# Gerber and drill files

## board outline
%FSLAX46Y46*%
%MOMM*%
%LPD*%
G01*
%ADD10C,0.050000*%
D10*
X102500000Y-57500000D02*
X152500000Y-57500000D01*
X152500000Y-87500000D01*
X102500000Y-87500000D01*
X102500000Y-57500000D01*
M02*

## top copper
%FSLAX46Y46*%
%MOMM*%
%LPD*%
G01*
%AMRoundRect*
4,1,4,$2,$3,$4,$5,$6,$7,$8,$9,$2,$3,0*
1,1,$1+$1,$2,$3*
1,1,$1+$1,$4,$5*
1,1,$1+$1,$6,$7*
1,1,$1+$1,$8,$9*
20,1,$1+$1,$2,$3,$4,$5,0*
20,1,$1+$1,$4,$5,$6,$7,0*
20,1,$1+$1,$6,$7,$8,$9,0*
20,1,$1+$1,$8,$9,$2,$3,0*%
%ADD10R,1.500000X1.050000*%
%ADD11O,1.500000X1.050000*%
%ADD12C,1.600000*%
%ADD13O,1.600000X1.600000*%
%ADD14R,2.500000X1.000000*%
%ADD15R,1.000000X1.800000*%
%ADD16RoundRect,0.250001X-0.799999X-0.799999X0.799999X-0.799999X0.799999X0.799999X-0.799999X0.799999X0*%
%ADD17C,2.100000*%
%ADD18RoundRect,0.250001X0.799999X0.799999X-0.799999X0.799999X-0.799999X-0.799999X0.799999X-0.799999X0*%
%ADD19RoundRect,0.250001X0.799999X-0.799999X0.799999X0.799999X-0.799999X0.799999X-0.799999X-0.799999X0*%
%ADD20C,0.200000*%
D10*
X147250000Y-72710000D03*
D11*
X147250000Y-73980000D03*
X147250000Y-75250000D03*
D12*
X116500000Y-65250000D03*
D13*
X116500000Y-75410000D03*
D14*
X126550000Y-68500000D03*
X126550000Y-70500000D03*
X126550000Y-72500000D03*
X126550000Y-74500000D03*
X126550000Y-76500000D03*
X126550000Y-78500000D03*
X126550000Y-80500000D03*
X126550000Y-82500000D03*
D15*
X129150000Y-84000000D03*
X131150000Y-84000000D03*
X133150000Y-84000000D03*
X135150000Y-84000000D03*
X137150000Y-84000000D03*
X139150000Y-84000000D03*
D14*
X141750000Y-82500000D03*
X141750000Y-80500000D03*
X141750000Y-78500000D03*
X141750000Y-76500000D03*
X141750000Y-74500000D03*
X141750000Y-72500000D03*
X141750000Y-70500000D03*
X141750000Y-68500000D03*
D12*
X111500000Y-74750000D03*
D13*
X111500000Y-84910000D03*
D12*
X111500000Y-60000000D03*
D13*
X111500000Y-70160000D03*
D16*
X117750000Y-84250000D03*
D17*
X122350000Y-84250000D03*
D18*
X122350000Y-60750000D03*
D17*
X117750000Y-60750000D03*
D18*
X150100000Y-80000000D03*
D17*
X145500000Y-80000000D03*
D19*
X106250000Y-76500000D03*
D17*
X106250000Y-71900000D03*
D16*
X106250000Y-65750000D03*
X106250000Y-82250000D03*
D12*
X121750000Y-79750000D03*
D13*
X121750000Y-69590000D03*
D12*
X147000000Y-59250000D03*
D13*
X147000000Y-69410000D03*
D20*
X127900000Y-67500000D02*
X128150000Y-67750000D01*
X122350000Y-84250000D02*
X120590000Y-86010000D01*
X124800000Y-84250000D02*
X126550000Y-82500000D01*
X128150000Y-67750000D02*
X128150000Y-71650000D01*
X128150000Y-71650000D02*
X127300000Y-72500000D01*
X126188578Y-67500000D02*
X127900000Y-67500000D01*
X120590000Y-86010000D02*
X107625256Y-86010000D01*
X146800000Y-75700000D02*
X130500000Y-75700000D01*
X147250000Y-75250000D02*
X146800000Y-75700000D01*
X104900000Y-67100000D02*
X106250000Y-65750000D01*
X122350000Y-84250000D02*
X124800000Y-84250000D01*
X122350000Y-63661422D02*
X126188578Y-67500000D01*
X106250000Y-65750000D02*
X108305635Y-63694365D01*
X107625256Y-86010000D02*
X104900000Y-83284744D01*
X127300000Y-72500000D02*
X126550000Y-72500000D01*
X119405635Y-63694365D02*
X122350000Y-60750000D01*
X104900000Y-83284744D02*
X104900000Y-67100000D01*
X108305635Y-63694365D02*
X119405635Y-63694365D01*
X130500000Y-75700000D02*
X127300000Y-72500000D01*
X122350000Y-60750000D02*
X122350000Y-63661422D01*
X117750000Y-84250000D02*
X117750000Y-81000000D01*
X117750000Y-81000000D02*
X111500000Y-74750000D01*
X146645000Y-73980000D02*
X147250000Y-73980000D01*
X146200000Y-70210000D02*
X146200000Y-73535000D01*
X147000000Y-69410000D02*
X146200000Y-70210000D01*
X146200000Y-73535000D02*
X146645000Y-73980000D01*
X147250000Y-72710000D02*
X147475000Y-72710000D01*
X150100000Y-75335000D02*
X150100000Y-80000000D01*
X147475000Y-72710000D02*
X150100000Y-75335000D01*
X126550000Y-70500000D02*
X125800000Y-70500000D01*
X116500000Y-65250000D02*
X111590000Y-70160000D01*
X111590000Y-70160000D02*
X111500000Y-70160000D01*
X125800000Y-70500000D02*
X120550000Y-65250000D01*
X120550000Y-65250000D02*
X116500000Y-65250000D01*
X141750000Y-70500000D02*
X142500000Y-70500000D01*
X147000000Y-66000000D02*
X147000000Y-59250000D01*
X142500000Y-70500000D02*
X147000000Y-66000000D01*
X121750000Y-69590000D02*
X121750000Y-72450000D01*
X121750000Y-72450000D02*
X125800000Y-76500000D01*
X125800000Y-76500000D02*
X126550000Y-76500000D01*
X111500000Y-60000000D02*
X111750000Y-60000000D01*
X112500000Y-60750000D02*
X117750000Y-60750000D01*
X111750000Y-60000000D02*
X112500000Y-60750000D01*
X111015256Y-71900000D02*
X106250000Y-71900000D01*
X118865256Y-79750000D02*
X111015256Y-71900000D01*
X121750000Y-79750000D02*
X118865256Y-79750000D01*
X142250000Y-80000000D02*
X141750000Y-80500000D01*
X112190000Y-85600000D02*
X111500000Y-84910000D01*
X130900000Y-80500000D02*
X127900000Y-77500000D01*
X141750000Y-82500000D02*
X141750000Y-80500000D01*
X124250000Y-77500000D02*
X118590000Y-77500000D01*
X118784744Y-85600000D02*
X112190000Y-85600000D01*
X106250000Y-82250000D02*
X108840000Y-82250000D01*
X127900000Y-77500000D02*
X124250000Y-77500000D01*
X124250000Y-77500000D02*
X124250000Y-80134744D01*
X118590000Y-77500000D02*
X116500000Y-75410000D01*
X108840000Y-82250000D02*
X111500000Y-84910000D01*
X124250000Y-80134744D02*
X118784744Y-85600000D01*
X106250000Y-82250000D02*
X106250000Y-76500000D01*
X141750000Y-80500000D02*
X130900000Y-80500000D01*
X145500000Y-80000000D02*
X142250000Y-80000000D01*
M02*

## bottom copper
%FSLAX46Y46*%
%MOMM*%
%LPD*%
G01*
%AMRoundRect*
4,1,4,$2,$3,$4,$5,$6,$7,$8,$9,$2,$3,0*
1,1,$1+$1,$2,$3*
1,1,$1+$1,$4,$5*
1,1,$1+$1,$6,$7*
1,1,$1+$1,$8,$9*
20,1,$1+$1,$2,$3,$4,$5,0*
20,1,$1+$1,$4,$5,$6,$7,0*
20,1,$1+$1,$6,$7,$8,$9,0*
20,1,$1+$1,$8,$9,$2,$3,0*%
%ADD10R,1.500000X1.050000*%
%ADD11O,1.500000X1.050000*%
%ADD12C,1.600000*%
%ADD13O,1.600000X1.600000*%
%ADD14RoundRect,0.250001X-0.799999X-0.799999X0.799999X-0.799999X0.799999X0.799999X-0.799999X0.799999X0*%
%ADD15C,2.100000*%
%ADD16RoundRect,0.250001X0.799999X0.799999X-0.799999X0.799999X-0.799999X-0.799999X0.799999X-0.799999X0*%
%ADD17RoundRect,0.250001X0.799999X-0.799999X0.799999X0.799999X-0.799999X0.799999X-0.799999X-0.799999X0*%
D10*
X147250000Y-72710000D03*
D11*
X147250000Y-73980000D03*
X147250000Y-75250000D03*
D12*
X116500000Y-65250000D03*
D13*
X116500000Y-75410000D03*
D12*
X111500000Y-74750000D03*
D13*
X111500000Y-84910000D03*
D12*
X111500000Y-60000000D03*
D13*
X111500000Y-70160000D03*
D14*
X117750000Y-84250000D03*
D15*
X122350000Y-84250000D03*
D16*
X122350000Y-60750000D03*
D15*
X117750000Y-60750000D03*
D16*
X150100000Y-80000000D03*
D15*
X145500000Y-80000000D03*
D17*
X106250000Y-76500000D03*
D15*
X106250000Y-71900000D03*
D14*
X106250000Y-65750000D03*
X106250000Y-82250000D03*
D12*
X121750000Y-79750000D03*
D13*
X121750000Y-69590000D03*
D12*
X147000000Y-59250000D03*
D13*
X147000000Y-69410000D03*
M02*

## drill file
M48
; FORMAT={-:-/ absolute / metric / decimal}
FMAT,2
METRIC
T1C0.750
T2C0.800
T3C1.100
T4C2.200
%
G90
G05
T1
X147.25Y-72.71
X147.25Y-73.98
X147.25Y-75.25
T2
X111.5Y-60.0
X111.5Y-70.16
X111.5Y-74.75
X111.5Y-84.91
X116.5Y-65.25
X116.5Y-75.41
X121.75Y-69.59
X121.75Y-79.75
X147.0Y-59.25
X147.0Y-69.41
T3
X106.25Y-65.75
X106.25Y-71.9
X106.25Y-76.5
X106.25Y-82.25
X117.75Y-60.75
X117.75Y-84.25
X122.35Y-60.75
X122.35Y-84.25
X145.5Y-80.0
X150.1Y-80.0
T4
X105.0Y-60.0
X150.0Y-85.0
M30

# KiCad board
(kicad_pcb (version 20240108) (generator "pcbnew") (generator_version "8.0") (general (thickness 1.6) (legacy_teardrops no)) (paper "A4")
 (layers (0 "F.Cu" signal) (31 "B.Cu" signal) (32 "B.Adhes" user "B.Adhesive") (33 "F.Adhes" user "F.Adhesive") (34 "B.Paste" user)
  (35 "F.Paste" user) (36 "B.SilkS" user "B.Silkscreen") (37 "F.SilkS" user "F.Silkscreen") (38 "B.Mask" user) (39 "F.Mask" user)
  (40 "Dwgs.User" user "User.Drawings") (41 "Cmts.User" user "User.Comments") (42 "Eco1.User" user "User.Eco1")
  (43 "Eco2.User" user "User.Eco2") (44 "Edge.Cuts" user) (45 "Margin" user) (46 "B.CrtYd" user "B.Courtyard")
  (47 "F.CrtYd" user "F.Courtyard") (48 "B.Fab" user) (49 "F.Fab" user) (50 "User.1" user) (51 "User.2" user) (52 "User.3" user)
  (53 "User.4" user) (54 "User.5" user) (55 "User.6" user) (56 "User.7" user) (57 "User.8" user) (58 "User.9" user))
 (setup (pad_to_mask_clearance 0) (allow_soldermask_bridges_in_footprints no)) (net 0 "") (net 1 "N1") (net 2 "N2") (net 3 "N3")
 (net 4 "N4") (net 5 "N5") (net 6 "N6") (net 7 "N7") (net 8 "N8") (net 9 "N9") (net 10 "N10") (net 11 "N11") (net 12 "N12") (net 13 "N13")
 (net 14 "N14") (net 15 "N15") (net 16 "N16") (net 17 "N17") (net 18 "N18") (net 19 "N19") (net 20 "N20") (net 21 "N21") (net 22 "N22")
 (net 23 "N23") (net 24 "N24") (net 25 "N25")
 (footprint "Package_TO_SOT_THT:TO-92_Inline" (layer "F.Cu") (at 147.25 72.71 -90)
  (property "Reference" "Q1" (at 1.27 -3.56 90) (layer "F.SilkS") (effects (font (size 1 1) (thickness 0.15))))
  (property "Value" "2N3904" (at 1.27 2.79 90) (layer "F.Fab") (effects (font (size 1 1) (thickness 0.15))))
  (pad "1" thru_hole rect (at 0 0 270) (size 1.05 1.5) (drill 0.75) (layers "*.Cu" "*.Mask") (remove_unused_layers no) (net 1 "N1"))
  (pad "2" thru_hole oval (at 1.27 0 270) (size 1.05 1.5) (drill 0.75) (layers "*.Cu" "*.Mask") (remove_unused_layers no) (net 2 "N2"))
  (pad "3" thru_hole oval (at 2.54 0 270) (size 1.05 1.5) (drill 0.75) (layers "*.Cu" "*.Mask") (remove_unused_layers no) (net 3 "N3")))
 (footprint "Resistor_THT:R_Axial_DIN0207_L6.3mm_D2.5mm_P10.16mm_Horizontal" (layer "F.Cu") (at 116.5 65.25 -90)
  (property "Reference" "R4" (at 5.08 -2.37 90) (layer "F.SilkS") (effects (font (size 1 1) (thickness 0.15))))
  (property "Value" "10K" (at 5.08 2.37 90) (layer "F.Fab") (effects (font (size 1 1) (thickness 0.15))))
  (pad "1" thru_hole circle (at 0 0 270) (size 1.6 1.6) (drill 0.8) (layers "*.Cu" "*.Mask") (remove_unused_layers no) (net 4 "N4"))
  (pad "2" thru_hole oval (at 10.16 0 270) (size 1.6 1.6) (drill 0.8) (layers "*.Cu" "*.Mask") (remove_unused_layers no) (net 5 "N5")))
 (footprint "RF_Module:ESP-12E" (layer "F.Cu") (at 134.15 72)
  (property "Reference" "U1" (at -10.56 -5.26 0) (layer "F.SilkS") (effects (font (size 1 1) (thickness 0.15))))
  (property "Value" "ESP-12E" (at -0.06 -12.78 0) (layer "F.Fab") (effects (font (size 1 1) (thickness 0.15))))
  (pad "1" smd rect (at -7.6 -3.5) (size 2.5 1) (layers "F.Cu" "F.Paste" "F.Mask") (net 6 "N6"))
  (pad "2" smd rect (at -7.6 -1.5) (size 2.5 1) (layers "F.Cu" "F.Paste" "F.Mask") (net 4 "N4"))
  (pad "3" smd rect (at -7.6 0.5) (size 2.5 1) (layers "F.Cu" "F.Paste" "F.Mask") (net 3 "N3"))
  (pad "4" smd rect (at -7.6 2.5) (size 2.5 1) (layers "F.Cu" "F.Paste" "F.Mask") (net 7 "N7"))
  (pad "5" smd rect (at -7.6 4.5) (size 2.5 1) (layers "F.Cu" "F.Paste" "F.Mask") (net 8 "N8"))
  (pad "6" smd rect (at -7.6 6.5) (size 2.5 1) (layers "F.Cu" "F.Paste" "F.Mask") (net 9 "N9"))
  (pad "7" smd rect (at -7.6 8.5) (size 2.5 1) (layers "F.Cu" "F.Paste" "F.Mask") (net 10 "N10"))
  (pad "8" smd rect (at -7.6 10.5) (size 2.5 1) (layers "F.Cu" "F.Paste" "F.Mask") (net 3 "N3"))
  (pad "9" smd rect (at -5 12) (size 1 1.8) (layers "F.Cu" "F.Paste" "F.Mask") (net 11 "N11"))
  (pad "10" smd rect (at -3 12) (size 1 1.8) (layers "F.Cu" "F.Paste" "F.Mask") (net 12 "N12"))
  (pad "11" smd rect (at -1 12) (size 1 1.8) (layers "F.Cu" "F.Paste" "F.Mask") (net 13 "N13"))
  (pad "12" smd rect (at 1 12) (size 1 1.8) (layers "F.Cu" "F.Paste" "F.Mask") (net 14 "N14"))
  (pad "13" smd rect (at 3 12) (size 1 1.8) (layers "F.Cu" "F.Paste" "F.Mask") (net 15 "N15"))
  (pad "14" smd rect (at 5 12) (size 1 1.8) (layers "F.Cu" "F.Paste" "F.Mask") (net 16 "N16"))
  (pad "15" smd rect (at 7.6 10.5) (size 2.5 1) (layers "F.Cu" "F.Paste" "F.Mask") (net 5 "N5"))
  (pad "16" smd rect (at 7.6 8.5) (size 2.5 1) (layers "F.Cu" "F.Paste" "F.Mask") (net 5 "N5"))
  (pad "17" smd rect (at 7.6 6.5) (size 2.5 1) (layers "F.Cu" "F.Paste" "F.Mask") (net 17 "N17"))
  (pad "18" smd rect (at 7.6 4.5) (size 2.5 1) (layers "F.Cu" "F.Paste" "F.Mask") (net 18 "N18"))
  (pad "19" smd rect (at 7.6 2.5) (size 2.5 1) (layers "F.Cu" "F.Paste" "F.Mask") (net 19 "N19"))
  (pad "20" smd rect (at 7.6 0.5) (size 2.5 1) (layers "F.Cu" "F.Paste" "F.Mask") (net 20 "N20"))
  (pad "21" smd rect (at 7.6 -1.5) (size 2.5 1) (layers "F.Cu" "F.Paste" "F.Mask") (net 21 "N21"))
  (pad "22" smd rect (at 7.6 -3.5) (size 2.5 1) (layers "F.Cu" "F.Paste" "F.Mask") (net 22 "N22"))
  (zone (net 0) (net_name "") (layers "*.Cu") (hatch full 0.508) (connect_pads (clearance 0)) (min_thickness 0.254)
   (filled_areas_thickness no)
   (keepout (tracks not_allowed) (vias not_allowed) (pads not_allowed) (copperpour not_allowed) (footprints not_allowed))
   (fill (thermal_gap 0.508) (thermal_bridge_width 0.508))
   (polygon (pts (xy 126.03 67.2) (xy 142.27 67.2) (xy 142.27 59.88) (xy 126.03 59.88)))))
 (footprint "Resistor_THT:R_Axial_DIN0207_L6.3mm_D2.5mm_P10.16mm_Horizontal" (layer "F.Cu") (at 111.5 74.75 -90)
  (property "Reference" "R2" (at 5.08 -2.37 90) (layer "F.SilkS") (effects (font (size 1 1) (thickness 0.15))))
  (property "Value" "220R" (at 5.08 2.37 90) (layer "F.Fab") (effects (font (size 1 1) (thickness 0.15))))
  (pad "1" thru_hole circle (at 0 0 270) (size 1.6 1.6) (drill 0.8) (layers "*.Cu" "*.Mask") (remove_unused_layers no) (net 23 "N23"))
  (pad "2" thru_hole oval (at 10.16 0 270) (size 1.6 1.6) (drill 0.8) (layers "*.Cu" "*.Mask") (remove_unused_layers no) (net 5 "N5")))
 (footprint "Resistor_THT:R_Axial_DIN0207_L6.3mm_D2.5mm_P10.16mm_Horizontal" (layer "F.Cu") (at 111.5 60 -90)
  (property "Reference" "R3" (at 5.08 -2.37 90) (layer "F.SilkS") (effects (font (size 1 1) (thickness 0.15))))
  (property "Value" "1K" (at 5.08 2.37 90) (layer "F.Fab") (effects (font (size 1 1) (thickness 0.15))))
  (pad "1" thru_hole circle (at 0 0 270) (size 1.6 1.6) (drill 0.8) (layers "*.Cu" "*.Mask") (remove_unused_layers no) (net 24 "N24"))
  (pad "2" thru_hole oval (at 10.16 0 270) (size 1.6 1.6) (drill 0.8) (layers "*.Cu" "*.Mask") (remove_unused_layers no) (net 4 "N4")))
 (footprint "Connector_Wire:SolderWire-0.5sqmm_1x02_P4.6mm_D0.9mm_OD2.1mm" (layer "F.Cu") (at 117.75 84.25)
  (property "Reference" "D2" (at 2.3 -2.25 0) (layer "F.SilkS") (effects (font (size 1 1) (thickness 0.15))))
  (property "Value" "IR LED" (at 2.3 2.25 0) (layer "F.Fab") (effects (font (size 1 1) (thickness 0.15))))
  (pad "1" thru_hole roundrect (at 0 0) (size 2.1 2.1) (drill 1.1) (layers "*.Cu" "*.Mask") (remove_unused_layers no)
   (roundrect_rratio 0.119048) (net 23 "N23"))
  (pad "2" thru_hole circle (at 4.6 0) (size 2.1 2.1) (drill 1.1) (layers "*.Cu" "*.Mask") (remove_unused_layers no) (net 3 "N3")))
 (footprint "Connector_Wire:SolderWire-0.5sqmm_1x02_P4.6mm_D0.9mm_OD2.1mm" (layer "F.Cu") (at 122.35 60.75 180)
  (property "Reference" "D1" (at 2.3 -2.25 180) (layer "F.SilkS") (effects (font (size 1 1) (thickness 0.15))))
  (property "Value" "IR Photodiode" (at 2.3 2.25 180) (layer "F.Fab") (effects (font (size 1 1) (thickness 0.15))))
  (pad "1" thru_hole roundrect (at 0 0 180) (size 2.1 2.1) (drill 1.1) (layers "*.Cu" "*.Mask") (remove_unused_layers no)
   (roundrect_rratio 0.119048) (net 3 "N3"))
  (pad "2" thru_hole circle (at 4.6 0 180) (size 2.1 2.1) (drill 1.1) (layers "*.Cu" "*.Mask") (remove_unused_layers no) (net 24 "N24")))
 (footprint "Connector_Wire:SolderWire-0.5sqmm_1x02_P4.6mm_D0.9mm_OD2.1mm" (layer "F.Cu") (at 150.1 80 180)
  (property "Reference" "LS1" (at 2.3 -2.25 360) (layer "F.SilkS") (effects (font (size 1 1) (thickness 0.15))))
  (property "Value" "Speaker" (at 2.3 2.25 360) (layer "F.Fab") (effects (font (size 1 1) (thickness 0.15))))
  (pad "1" thru_hole roundrect (at 0 0 180) (size 2.1 2.1) (drill 1.1) (layers "*.Cu" "*.Mask") (remove_unused_layers no)
   (roundrect_rratio 0.119048) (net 1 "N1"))
  (pad "2" thru_hole circle (at 4.6 0 180) (size 2.1 2.1) (drill 1.1) (layers "*.Cu" "*.Mask") (remove_unused_layers no) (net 5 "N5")))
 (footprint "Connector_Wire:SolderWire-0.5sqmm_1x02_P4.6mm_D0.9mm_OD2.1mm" (layer "F.Cu") (at 106.25 76.5 90)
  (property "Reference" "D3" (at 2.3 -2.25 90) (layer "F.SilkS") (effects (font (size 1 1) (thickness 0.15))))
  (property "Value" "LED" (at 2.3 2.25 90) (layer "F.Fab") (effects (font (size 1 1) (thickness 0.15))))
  (pad "1" thru_hole roundrect (at 0 0 90) (size 2.1 2.1) (drill 1.1) (layers "*.Cu" "*.Mask") (remove_unused_layers no)
   (roundrect_rratio 0.119048) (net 5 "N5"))
  (pad "2" thru_hole circle (at 4.6 0 90) (size 2.1 2.1) (drill 1.1) (layers "*.Cu" "*.Mask") (remove_unused_layers no) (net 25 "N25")))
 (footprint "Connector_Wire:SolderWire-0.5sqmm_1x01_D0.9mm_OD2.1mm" (layer "F.Cu") (at 106.25 65.75)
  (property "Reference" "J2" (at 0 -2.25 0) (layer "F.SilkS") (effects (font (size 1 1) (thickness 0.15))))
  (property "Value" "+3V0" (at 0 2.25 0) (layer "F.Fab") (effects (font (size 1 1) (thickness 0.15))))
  (pad "1" thru_hole roundrect (at 0 0) (size 2.1 2.1) (drill 1.1) (layers "*.Cu" "*.Mask") (remove_unused_layers no)
   (roundrect_rratio 0.119048) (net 3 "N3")))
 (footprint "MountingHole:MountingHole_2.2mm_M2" (layer "F.Cu") (at 150 85)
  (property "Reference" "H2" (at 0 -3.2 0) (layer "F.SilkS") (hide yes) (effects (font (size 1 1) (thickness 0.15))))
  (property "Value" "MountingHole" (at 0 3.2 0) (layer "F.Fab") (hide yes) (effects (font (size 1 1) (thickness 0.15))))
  (pad "" np_thru_hole circle (at 0 0) (size 2.2 2.2) (drill 2.2) (layers "*.Cu" "*.Mask")))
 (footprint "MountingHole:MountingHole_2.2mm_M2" (layer "F.Cu") (at 105 60)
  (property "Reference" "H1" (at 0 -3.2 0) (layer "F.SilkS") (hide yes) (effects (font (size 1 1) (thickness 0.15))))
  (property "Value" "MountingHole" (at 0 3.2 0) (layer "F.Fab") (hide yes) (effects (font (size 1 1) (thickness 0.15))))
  (pad "" np_thru_hole circle (at 0 0) (size 2.2 2.2) (drill 2.2) (layers "*.Cu" "*.Mask")))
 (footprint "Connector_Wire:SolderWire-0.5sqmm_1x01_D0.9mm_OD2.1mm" (layer "F.Cu") (at 106.25 82.25)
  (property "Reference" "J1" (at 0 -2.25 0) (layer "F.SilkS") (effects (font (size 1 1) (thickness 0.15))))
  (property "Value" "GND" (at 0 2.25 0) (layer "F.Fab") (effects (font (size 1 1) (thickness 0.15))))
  (pad "1" thru_hole roundrect (at 0 0) (size 2.1 2.1) (drill 1.1) (layers "*.Cu" "*.Mask") (remove_unused_layers no)
   (roundrect_rratio 0.119048) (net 5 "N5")))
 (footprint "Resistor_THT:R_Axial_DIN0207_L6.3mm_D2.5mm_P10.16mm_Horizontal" (layer "F.Cu") (at 121.75 79.75 90)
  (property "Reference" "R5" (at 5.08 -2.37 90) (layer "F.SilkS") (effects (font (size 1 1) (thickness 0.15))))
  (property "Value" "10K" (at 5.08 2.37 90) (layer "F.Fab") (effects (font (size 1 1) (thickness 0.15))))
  (pad "1" thru_hole circle (at 0 0 90) (size 1.6 1.6) (drill 0.8) (layers "*.Cu" "*.Mask") (remove_unused_layers no) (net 25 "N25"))
  (pad "2" thru_hole oval (at 10.16 0 90) (size 1.6 1.6) (drill 0.8) (layers "*.Cu" "*.Mask") (remove_unused_layers no) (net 8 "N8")))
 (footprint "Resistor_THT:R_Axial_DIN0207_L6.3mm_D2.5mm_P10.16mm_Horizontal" (layer "F.Cu") (at 147 59.25 -90)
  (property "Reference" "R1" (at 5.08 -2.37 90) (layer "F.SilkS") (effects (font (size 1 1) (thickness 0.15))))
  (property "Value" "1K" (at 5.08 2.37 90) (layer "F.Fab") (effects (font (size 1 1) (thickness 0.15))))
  (pad "1" thru_hole circle (at 0 0 270) (size 1.6 1.6) (drill 0.8) (layers "*.Cu" "*.Mask") (remove_unused_layers no) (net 21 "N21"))
  (pad "2" thru_hole oval (at 10.16 0 270) (size 1.6 1.6) (drill 0.8) (layers "*.Cu" "*.Mask") (remove_unused_layers no) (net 2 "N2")))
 (gr_rect (start 102.5 57.5) (end 152.5 87.5) (stroke (width 0.05) (type default)) (fill none) (layer "Edge.Cuts"))
 (segment (start 127.9 67.5) (end 128.15 67.75) (width 0.2) (layer "F.Cu") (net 3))
 (segment (start 122.35 84.25) (end 120.59 86.01) (width 0.2) (layer "F.Cu") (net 3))
 (segment (start 124.8 84.25) (end 126.55 82.5) (width 0.2) (layer "F.Cu") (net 3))
 (segment (start 128.15 67.75) (end 128.15 71.65) (width 0.2) (layer "F.Cu") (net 3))
 (segment (start 128.15 71.65) (end 127.3 72.5) (width 0.2) (layer "F.Cu") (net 3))
 (segment (start 126.188578 67.5) (end 127.9 67.5) (width 0.2) (layer "F.Cu") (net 3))
 (segment (start 120.59 86.01) (end 107.625256 86.01) (width 0.2) (layer "F.Cu") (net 3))
 (segment (start 146.8 75.7) (end 130.5 75.7) (width 0.2) (layer "F.Cu") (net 3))
 (segment (start 147.25 75.25) (end 146.8 75.7) (width 0.2) (layer "F.Cu") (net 3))
 (segment (start 104.9 67.1) (end 106.25 65.75) (width 0.2) (layer "F.Cu") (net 3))
 (segment (start 122.35 84.25) (end 124.8 84.25) (width 0.2) (layer "F.Cu") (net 3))
 (segment (start 122.35 63.661422) (end 126.188578 67.5) (width 0.2) (layer "F.Cu") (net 3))
 (segment (start 106.25 65.75) (end 108.305635 63.694365) (width 0.2) (layer "F.Cu") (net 3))
 (segment (start 107.625256 86.01) (end 104.9 83.284744) (width 0.2) (layer "F.Cu") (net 3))
 (segment (start 127.3 72.5) (end 126.55 72.5) (width 0.2) (layer "F.Cu") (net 3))
 (segment (start 119.405635 63.694365) (end 122.35 60.75) (width 0.2) (layer "F.Cu") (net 3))
 (segment (start 104.9 83.284744) (end 104.9 67.1) (width 0.2) (layer "F.Cu") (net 3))
 (segment (start 108.305635 63.694365) (end 119.405635 63.694365) (width 0.2) (layer "F.Cu") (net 3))
 (segment (start 130.5 75.7) (end 127.3 72.5) (width 0.2) (layer "F.Cu") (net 3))
 (segment (start 122.35 60.75) (end 122.35 63.661422) (width 0.2) (layer "F.Cu") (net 3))
 (segment (start 117.75 84.25) (end 117.75 81) (width 0.2) (layer "F.Cu") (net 23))
 (segment (start 117.75 81) (end 111.5 74.75) (width 0.2) (layer "F.Cu") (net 23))
 (segment (start 146.645 73.98) (end 147.25 73.98) (width 0.2) (layer "F.Cu") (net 2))
 (segment (start 146.2 70.21) (end 146.2 73.535) (width 0.2) (layer "F.Cu") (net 2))
 (segment (start 147 69.41) (end 146.2 70.21) (width 0.2) (layer "F.Cu") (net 2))
 (segment (start 146.2 73.535) (end 146.645 73.98) (width 0.2) (layer "F.Cu") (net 2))
 (segment (start 147.25 72.71) (end 147.475 72.71) (width 0.2) (layer "F.Cu") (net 1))
 (segment (start 150.1 75.335) (end 150.1 80) (width 0.2) (layer "F.Cu") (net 1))
 (segment (start 147.475 72.71) (end 150.1 75.335) (width 0.2) (layer "F.Cu") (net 1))
 (segment (start 126.55 70.5) (end 125.8 70.5) (width 0.2) (layer "F.Cu") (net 4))
 (segment (start 116.5 65.25) (end 111.59 70.16) (width 0.2) (layer "F.Cu") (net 4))
 (segment (start 111.59 70.16) (end 111.5 70.16) (width 0.2) (layer "F.Cu") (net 4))
 (segment (start 125.8 70.5) (end 120.55 65.25) (width 0.2) (layer "F.Cu") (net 4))
 (segment (start 120.55 65.25) (end 116.5 65.25) (width 0.2) (layer "F.Cu") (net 4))
 (segment (start 141.75 70.5) (end 142.5 70.5) (width 0.2) (layer "F.Cu") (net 21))
 (segment (start 147 66) (end 147 59.25) (width 0.2) (layer "F.Cu") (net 21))
 (segment (start 142.5 70.5) (end 147 66) (width 0.2) (layer "F.Cu") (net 21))
 (segment (start 121.75 69.59) (end 121.75 72.45) (width 0.2) (layer "F.Cu") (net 8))
 (segment (start 121.75 72.45) (end 125.8 76.5) (width 0.2) (layer "F.Cu") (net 8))
 (segment (start 125.8 76.5) (end 126.55 76.5) (width 0.2) (layer "F.Cu") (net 8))
 (segment (start 111.5 60) (end 111.75 60) (width 0.2) (layer "F.Cu") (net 24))
 (segment (start 112.5 60.75) (end 117.75 60.75) (width 0.2) (layer "F.Cu") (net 24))
 (segment (start 111.75 60) (end 112.5 60.75) (width 0.2) (layer "F.Cu") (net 24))
 (segment (start 111.015256 71.9) (end 106.25 71.9) (width 0.2) (layer "F.Cu") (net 25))
 (segment (start 118.865256 79.75) (end 111.015256 71.9) (width 0.2) (layer "F.Cu") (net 25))
 (segment (start 121.75 79.75) (end 118.865256 79.75) (width 0.2) (layer "F.Cu") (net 25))
 (segment (start 142.25 80) (end 141.75 80.5) (width 0.2) (layer "F.Cu") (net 5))
 (segment (start 112.19 85.6) (end 111.5 84.91) (width 0.2) (layer "F.Cu") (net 5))
 (segment (start 130.9 80.5) (end 127.9 77.5) (width 0.2) (layer "F.Cu") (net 5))
 (segment (start 141.75 82.5) (end 141.75 80.5) (width 0.2) (layer "F.Cu") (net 5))
 (segment (start 124.25 77.5) (end 118.59 77.5) (width 0.2) (layer "F.Cu") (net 5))
 (segment (start 118.784744 85.6) (end 112.19 85.6) (width 0.2) (layer "F.Cu") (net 5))
 (segment (start 106.25 82.25) (end 108.84 82.25) (width 0.2) (layer "F.Cu") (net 5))
 (segment (start 127.9 77.5) (end 124.25 77.5) (width 0.2) (layer "F.Cu") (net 5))
 (segment (start 124.25 77.5) (end 124.25 80.134744) (width 0.2) (layer "F.Cu") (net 5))
 (segment (start 118.59 77.5) (end 116.5 75.41) (width 0.2) (layer "F.Cu") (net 5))
 (segment (start 108.84 82.25) (end 111.5 84.91) (width 0.2) (layer "F.Cu") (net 5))
 (segment (start 124.25 80.134744) (end 118.784744 85.6) (width 0.2) (layer "F.Cu") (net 5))
 (segment (start 106.25 82.25) (end 106.25 76.5) (width 0.2) (layer "F.Cu") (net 5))
 (segment (start 141.75 80.5) (end 130.9 80.5) (width 0.2) (layer "F.Cu") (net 5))
 (segment (start 145.5 80) (end 142.25 80) (width 0.2) (layer "F.Cu") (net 5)))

